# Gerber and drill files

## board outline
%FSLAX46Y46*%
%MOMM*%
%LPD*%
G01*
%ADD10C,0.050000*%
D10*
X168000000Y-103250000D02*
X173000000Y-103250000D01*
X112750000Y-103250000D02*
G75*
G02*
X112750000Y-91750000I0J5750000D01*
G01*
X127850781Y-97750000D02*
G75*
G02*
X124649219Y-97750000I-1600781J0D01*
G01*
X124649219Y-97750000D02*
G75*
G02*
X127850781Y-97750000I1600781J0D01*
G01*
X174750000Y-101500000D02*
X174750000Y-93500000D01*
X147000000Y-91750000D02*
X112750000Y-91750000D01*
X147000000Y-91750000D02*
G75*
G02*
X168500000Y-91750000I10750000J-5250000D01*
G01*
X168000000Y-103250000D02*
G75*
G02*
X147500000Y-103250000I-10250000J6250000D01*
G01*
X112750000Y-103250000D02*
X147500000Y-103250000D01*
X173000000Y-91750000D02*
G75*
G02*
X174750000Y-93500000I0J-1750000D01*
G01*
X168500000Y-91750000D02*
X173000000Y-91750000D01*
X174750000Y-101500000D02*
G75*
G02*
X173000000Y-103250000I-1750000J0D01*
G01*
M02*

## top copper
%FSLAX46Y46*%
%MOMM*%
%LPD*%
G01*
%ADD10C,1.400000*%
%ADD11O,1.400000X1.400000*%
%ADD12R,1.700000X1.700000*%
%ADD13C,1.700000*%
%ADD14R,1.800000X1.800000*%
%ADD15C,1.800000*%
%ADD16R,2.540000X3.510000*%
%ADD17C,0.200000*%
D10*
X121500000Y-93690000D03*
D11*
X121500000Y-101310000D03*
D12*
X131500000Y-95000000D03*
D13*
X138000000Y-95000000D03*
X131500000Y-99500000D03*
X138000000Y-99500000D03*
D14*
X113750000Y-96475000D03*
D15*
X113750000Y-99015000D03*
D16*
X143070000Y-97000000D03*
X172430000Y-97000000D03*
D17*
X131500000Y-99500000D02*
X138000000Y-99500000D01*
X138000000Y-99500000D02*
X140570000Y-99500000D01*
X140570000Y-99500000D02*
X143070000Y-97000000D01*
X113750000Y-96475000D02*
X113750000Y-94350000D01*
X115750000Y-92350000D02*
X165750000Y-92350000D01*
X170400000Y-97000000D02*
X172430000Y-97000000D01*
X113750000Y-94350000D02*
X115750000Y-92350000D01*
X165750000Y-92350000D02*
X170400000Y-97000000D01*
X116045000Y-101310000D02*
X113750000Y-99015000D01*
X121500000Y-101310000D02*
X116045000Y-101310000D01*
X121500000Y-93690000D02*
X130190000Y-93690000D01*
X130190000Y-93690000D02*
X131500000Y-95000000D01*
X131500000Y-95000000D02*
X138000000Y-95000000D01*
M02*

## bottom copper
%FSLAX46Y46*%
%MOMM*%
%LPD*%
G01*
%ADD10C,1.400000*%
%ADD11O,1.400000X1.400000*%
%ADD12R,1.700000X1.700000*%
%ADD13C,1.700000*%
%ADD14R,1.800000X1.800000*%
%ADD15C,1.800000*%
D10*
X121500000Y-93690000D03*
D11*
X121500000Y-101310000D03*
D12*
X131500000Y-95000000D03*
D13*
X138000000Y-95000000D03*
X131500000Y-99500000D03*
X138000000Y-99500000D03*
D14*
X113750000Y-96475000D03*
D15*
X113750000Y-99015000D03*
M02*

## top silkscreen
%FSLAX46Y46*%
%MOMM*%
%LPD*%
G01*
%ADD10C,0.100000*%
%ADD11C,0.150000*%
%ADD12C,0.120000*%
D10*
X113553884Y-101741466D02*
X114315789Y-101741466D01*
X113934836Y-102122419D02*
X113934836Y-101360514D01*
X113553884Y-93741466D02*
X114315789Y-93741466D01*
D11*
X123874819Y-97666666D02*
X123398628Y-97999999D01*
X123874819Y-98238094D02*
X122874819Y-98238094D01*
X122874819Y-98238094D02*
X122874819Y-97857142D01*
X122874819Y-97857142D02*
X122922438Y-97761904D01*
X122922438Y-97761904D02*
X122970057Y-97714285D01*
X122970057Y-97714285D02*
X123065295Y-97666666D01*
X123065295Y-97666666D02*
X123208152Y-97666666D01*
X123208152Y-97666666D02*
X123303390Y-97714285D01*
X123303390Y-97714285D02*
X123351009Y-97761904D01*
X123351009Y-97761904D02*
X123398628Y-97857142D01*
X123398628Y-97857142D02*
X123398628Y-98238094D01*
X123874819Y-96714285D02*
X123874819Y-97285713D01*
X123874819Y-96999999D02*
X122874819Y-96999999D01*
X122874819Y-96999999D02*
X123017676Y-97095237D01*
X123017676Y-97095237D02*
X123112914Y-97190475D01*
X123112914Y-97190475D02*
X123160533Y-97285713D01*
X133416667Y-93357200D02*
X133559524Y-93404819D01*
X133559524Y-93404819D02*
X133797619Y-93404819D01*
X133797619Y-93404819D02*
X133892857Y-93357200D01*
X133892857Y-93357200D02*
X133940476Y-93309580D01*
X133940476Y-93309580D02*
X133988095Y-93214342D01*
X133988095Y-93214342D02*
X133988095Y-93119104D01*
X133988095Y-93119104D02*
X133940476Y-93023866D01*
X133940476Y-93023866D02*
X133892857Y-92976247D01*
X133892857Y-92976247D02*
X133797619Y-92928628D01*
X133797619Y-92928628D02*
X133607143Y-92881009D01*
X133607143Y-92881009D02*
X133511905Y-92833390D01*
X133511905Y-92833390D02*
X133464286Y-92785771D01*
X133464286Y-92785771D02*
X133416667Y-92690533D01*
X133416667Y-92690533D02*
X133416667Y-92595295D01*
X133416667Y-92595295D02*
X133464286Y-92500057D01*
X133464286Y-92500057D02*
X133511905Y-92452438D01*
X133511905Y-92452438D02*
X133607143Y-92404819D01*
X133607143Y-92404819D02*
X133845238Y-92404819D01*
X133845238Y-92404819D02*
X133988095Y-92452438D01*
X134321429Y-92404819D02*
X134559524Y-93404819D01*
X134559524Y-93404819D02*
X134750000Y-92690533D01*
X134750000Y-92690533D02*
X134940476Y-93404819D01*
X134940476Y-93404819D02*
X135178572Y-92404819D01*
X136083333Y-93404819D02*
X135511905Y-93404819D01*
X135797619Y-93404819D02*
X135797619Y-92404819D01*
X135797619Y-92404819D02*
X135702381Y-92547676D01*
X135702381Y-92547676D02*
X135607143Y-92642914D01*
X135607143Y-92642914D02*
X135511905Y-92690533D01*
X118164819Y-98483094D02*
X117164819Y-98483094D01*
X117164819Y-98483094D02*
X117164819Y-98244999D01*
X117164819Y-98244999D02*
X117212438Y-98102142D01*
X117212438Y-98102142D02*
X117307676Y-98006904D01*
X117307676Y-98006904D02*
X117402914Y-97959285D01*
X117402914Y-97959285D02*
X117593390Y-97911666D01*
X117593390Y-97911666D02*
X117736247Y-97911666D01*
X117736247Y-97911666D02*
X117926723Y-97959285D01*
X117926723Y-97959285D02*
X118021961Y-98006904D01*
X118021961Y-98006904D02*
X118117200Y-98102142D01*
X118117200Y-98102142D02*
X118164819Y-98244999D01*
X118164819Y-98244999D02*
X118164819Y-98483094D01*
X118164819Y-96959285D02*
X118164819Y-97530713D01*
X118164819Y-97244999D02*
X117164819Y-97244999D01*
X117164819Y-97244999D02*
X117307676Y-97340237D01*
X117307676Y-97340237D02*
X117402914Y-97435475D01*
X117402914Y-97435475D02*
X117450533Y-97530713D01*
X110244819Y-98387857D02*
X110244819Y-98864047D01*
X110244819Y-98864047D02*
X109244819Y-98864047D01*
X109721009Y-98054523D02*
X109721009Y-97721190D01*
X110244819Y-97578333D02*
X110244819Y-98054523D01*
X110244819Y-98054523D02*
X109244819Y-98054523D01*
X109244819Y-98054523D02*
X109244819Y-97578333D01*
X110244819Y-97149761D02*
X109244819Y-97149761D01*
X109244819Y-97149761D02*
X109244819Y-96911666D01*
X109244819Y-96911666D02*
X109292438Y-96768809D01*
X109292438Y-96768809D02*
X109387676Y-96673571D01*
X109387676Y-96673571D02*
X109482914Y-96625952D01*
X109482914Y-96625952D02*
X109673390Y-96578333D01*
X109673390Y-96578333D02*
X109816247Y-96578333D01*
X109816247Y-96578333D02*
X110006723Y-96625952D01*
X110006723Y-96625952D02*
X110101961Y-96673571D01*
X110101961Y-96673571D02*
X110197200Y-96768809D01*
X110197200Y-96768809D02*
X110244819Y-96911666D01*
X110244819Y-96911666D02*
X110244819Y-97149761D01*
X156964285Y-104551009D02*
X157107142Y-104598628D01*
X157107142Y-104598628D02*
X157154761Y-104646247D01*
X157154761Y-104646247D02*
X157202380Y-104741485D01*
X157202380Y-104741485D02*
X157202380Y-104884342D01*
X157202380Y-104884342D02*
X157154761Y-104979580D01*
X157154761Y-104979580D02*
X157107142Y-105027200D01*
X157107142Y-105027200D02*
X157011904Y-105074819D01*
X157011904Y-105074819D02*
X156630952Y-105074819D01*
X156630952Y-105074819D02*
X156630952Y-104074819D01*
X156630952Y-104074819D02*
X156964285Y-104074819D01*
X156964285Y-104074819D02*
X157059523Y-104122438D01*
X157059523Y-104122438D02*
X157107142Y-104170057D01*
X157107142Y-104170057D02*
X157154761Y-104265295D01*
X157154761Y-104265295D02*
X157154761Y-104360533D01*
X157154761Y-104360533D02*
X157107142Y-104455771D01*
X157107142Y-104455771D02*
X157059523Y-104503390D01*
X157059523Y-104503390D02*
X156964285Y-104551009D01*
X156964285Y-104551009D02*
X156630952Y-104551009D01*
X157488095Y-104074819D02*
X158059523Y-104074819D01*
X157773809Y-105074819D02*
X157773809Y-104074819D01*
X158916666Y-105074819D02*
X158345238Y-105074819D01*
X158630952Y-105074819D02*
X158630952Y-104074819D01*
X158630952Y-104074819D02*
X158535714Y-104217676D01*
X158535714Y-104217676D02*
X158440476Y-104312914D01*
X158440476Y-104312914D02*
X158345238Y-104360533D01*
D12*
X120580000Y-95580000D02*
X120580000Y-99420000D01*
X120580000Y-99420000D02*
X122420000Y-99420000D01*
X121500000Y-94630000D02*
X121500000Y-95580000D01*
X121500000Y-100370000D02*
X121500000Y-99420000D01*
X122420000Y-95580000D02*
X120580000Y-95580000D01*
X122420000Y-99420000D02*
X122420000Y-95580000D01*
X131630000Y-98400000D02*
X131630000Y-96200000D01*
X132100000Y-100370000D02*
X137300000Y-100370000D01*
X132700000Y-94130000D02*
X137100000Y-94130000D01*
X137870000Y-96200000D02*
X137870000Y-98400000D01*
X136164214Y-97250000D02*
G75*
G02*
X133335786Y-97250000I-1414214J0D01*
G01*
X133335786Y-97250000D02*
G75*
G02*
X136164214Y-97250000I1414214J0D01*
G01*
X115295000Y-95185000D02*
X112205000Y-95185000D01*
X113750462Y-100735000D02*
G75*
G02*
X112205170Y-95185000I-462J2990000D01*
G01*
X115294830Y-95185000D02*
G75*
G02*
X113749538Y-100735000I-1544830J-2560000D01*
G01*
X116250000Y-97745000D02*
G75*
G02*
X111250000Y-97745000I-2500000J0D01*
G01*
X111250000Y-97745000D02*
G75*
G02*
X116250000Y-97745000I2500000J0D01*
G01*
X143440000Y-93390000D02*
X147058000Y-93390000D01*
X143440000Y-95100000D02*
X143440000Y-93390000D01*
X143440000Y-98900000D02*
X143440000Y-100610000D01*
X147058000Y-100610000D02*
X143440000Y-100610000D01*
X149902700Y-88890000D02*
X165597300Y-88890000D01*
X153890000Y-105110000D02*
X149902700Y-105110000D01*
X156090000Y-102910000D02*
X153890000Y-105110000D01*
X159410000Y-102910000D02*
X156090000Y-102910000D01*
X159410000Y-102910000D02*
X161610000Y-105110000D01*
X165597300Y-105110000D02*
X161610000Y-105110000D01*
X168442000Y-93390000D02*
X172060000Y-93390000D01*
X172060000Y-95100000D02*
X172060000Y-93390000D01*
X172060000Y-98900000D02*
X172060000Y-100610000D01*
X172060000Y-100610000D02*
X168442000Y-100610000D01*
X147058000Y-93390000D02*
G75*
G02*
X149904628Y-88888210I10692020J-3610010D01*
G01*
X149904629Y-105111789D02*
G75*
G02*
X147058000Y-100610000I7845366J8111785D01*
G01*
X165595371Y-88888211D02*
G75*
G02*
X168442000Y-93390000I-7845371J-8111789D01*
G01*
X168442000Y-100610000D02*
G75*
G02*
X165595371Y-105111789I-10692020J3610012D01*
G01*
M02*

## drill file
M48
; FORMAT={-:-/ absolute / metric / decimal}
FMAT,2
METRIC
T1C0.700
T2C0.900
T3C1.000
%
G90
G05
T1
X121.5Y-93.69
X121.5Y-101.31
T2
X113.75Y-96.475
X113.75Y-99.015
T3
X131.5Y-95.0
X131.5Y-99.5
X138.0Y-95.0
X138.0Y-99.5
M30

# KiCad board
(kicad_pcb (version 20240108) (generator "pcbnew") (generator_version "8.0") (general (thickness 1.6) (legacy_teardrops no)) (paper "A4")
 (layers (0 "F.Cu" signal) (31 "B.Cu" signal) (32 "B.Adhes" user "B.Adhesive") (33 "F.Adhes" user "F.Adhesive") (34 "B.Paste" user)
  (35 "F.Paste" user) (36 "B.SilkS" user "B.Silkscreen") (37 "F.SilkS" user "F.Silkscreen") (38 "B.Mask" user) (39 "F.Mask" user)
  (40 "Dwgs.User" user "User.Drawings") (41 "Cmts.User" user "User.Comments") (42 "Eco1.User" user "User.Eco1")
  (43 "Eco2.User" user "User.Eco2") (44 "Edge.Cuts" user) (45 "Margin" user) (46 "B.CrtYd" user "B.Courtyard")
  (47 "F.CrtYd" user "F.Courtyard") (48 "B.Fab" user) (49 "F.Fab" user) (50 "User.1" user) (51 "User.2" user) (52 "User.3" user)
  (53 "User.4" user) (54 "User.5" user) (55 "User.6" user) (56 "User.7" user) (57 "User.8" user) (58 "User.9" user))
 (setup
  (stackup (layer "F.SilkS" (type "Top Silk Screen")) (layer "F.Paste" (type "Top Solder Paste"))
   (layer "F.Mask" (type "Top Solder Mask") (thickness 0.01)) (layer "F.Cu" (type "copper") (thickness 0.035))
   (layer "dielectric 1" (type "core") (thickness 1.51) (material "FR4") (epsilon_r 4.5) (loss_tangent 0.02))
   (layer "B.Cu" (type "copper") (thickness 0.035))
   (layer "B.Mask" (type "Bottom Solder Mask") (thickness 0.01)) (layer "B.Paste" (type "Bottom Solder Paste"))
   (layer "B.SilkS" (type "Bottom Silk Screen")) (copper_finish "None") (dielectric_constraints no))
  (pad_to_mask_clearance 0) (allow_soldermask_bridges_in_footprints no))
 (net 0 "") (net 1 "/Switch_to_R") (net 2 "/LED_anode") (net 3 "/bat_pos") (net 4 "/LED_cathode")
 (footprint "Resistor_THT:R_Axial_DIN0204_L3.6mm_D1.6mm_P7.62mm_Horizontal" (layer "F.Cu") (at 121.5 93.69 -90)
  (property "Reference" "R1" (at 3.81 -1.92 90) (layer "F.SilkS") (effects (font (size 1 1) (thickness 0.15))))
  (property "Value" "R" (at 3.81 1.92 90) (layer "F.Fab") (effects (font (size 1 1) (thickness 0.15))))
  (fp_line (start 1.89 0.92) (end 5.73 0.92) (stroke (width 0.12) (type solid)) (layer "F.SilkS"))
  (fp_line (start 5.73 0.92) (end 5.73 -0.92) (stroke (width 0.12) (type solid)) (layer "F.SilkS"))
  (fp_line (start 0.94 0) (end 1.89 0) (stroke (width 0.12) (type solid)) (layer "F.SilkS"))
  (fp_line (start 6.68 0) (end 5.73 0) (stroke (width 0.12) (type solid)) (layer "F.SilkS"))
  (fp_line (start 1.89 -0.92) (end 1.89 0.92) (stroke (width 0.12) (type solid)) (layer "F.SilkS"))
  (fp_line (start 5.73 -0.92) (end 1.89 -0.92) (stroke (width 0.12) (type solid)) (layer "F.SilkS"))
  (pad "1" thru_hole circle (at 0 0 270) (size 1.4 1.4) (drill 0.7) (layers "*.Cu" "*.Mask") (remove_unused_layers no)
   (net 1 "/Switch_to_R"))
  (pad "2" thru_hole oval (at 7.62 0 270) (size 1.4 1.4) (drill 0.7) (layers "*.Cu" "*.Mask") (remove_unused_layers no) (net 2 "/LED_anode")))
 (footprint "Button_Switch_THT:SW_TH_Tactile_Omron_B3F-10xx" (layer "F.Cu") (at 131.5 95)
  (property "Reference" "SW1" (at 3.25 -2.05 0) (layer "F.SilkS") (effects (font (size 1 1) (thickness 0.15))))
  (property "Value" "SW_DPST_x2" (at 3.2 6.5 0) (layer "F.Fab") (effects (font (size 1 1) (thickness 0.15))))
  (fp_line (start 0.13 3.4) (end 0.13 1.2) (stroke (width 0.12) (type solid)) (layer "F.SilkS"))
  (fp_line (start 0.6 5.37) (end 5.8 5.37) (stroke (width 0.12) (type solid)) (layer "F.SilkS"))
  (fp_line (start 1.2 -0.87) (end 5.6 -0.87) (stroke (width 0.12) (type solid)) (layer "F.SilkS"))
  (fp_line (start 6.37 1.2) (end 6.37 3.4) (stroke (width 0.12) (type solid)) (layer "F.SilkS"))
  (fp_circle (center 3.25 2.25) (end 4.25 3.25) (stroke (width 0.12) (type solid)) (fill none) (layer "F.SilkS"))
  (pad "1" thru_hole rect (at 0 0) (size 1.7 1.7) (drill 1) (layers "*.Cu" "*.Mask") (remove_unused_layers no) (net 1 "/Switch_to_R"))
  (pad "1" thru_hole circle (at 6.5 0) (size 1.7 1.7) (drill 1) (layers "*.Cu" "*.Mask") (remove_unused_layers no) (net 1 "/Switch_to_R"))
  (pad "2" thru_hole circle (at 0 4.5) (size 1.7 1.7) (drill 1) (layers "*.Cu" "*.Mask") (remove_unused_layers no) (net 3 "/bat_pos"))
  (pad "2" thru_hole circle (at 6.5 4.5) (size 1.7 1.7) (drill 1) (layers "*.Cu" "*.Mask") (remove_unused_layers no) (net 3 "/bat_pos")))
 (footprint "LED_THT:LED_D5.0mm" (layer "F.Cu") (at 113.75 96.475 -90)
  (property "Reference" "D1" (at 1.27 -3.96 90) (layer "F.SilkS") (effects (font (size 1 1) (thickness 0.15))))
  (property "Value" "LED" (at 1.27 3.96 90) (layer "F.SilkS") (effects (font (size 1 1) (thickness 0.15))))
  (fp_line (start -1.29 -1.545) (end -1.29 1.545) (stroke (width 0.12) (type solid)) (layer "F.SilkS"))
  (fp_arc (start 4.26 -0.000462) (mid 2.072002 2.880433) (end -1.29 1.54483) (stroke (width 0.12) (type solid)) (layer "F.SilkS"))
  (fp_arc (start -1.29 -1.54483) (mid 2.072002 -2.880433) (end 4.26 0.000462) (stroke (width 0.12) (type solid)) (layer "F.SilkS"))
  (fp_circle (center 1.27 0) (end 3.77 0) (stroke (width 0.12) (type solid)) (fill none) (layer "F.SilkS"))
  (pad "1" thru_hole rect (at 0 0 270) (size 1.8 1.8) (drill 0.9) (layers "*.Cu" "*.Mask") (remove_unused_layers no) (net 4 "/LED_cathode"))
  (pad "2" thru_hole circle (at 2.54 0 270) (size 1.8 1.8) (drill 0.9) (layers "*.Cu" "*.Mask") (remove_unused_layers no)
   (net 2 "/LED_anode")))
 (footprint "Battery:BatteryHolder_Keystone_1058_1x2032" (layer "F.Cu") (at 157.75 97)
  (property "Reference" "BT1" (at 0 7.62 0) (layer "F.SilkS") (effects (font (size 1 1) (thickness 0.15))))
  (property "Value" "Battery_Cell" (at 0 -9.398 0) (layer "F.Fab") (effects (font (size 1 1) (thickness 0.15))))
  (fp_line (start -14.31 -3.61) (end -10.692 -3.61) (stroke (width 0.12) (type solid)) (layer "F.SilkS"))
  (fp_line (start -14.31 -1.9) (end -14.31 -3.61) (stroke (width 0.12) (type solid)) (layer "F.SilkS"))
  (fp_line (start -14.31 1.9) (end -14.31 3.61) (stroke (width 0.12) (type solid)) (layer "F.SilkS"))
  (fp_line (start -10.692 3.61) (end -14.31 3.61) (stroke (width 0.12) (type solid)) (layer "F.SilkS"))
  (fp_line (start -7.8473 -8.11) (end 7.8473 -8.11) (stroke (width 0.12) (type solid)) (layer "F.SilkS"))
  (fp_line (start -3.86 8.11) (end -7.8473 8.11) (stroke (width 0.12) (type solid)) (layer "F.SilkS"))
  (fp_line (start -1.66 5.91) (end -3.86 8.11) (stroke (width 0.12) (type solid)) (layer "F.SilkS"))
  (fp_line (start 1.66 5.91) (end -1.66 5.91) (stroke (width 0.12) (type solid)) (layer "F.SilkS"))
  (fp_line (start 1.66 5.91) (end 3.86 8.11) (stroke (width 0.12) (type solid)) (layer "F.SilkS"))
  (fp_line (start 7.8473 8.11) (end 3.86 8.11) (stroke (width 0.12) (type solid)) (layer "F.SilkS"))
  (fp_line (start 10.692 -3.61) (end 14.31 -3.61) (stroke (width 0.12) (type solid)) (layer "F.SilkS"))
  (fp_line (start 14.31 -1.9) (end 14.31 -3.61) (stroke (width 0.12) (type solid)) (layer "F.SilkS"))
  (fp_line (start 14.31 1.9) (end 14.31 3.61) (stroke (width 0.12) (type solid)) (layer "F.SilkS"))
  (fp_line (start 14.31 3.61) (end 10.692 3.61) (stroke (width 0.12) (type solid)) (layer "F.SilkS"))
  (fp_arc (start -10.692 -3.61) (mid -9.538084 -6.031244) (end -7.845371 -8.111789) (stroke (width 0.12) (type solid)) (layer "F.SilkS"))
  (fp_arc (start -7.845371 8.111789) (mid -9.538085 6.031244) (end -10.692 3.61) (stroke (width 0.12) (type solid)) (layer "F.SilkS"))
  (fp_arc (start 7.845371 -8.111789) (mid 9.538085 -6.031244) (end 10.692 -3.61) (stroke (width 0.12) (type solid)) (layer "F.SilkS"))
  (fp_arc (start 10.692 3.61) (mid 9.538084 6.031244) (end 7.845371 8.111789) (stroke (width 0.12) (type solid)) (layer "F.SilkS"))
  (pad "1" smd rect (at -14.68 0) (size 2.54 3.51) (layers "F.Cu" "F.Paste" "F.Mask") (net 3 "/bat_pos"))
  (pad "2" smd rect (at 14.68 0) (size 2.54 3.51) (layers "F.Cu" "F.Paste" "F.Mask") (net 4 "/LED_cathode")))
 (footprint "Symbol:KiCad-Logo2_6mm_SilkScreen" (layer "B.Cu") (at 157.5 96.25 180)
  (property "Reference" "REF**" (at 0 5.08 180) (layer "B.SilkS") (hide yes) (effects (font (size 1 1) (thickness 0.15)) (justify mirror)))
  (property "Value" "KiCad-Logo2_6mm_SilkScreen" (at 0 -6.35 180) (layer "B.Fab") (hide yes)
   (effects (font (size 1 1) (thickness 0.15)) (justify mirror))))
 (gr_line (start 168 103.25) (end 173 103.25) (stroke (width 0.05) (type default)) (layer "Edge.Cuts"))
 (gr_arc (start 112.75 103.25) (mid 107 97.5) (end 112.75 91.75) (stroke (width 0.05) (type default)) (layer "Edge.Cuts"))
 (gr_circle (center 126.25 97.75) (end 127.5 98.75) (stroke (width 0.05) (type default)) (fill none) (layer "Edge.Cuts"))
 (gr_line (start 174.75 101.5) (end 174.75 93.5) (stroke (width 0.05) (type default)) (layer "Edge.Cuts"))
 (gr_line (start 147 91.75) (end 112.75 91.75) (stroke (width 0.05) (type default)) (layer "Edge.Cuts"))
 (gr_arc (start 147 91.75) (mid 157.75 85.036514) (end 168.5 91.75) (stroke (width 0.05) (type default)) (layer "Edge.Cuts"))
 (gr_arc (start 168 103.25) (mid 157.75 109.005207) (end 147.5 103.25) (stroke (width 0.05) (type default)) (layer "Edge.Cuts"))
 (gr_line (start 112.75 103.25) (end 147.5 103.25) (stroke (width 0.05) (type default)) (layer "Edge.Cuts"))
 (gr_arc (start 173 91.75) (mid 174.237437 92.262563) (end 174.75 93.5) (stroke (width 0.05) (type default)) (layer "Edge.Cuts"))
 (gr_line (start 168.5 91.75) (end 173 91.75) (stroke (width 0.05) (type default)) (layer "Edge.Cuts"))
 (gr_arc (start 174.75 101.5) (mid 174.237437 102.737437) (end 173 103.25) (stroke (width 0.05) (type default)) (layer "Edge.Cuts"))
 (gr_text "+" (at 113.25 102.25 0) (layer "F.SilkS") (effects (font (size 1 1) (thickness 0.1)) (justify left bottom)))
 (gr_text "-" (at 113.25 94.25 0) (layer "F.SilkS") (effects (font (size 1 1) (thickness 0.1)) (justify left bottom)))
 (segment (start 131.5 99.5) (end 138 99.5) (width 0.2) (layer "F.Cu") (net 3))
 (segment (start 138 99.5) (end 140.57 99.5) (width 0.2) (layer "F.Cu") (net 3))
 (segment (start 140.57 99.5) (end 143.07 97) (width 0.2) (layer "F.Cu") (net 3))
 (segment (start 113.75 96.475) (end 113.75 94.35) (width 0.2) (layer "F.Cu") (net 4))
 (segment (start 115.75 92.35) (end 165.75 92.35) (width 0.2) (layer "F.Cu") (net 4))
 (segment (start 170.4 97) (end 172.43 97) (width 0.2) (layer "F.Cu") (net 4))
 (segment (start 113.75 94.35) (end 115.75 92.35) (width 0.2) (layer "F.Cu") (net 4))
 (segment (start 165.75 92.35) (end 170.4 97) (width 0.2) (layer "F.Cu") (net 4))
 (segment (start 116.045 101.31) (end 113.75 99.015) (width 0.2) (layer "F.Cu") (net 2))
 (segment (start 121.5 101.31) (end 116.045 101.31) (width 0.2) (layer "F.Cu") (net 2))
 (segment (start 121.5 93.69) (end 130.19 93.69) (width 0.2) (layer "F.Cu") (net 1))
 (segment (start 130.19 93.69) (end 131.5 95) (width 0.2) (layer "F.Cu") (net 1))
 (segment (start 131.5 95) (end 138 95) (width 0.2) (layer "F.Cu") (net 1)))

